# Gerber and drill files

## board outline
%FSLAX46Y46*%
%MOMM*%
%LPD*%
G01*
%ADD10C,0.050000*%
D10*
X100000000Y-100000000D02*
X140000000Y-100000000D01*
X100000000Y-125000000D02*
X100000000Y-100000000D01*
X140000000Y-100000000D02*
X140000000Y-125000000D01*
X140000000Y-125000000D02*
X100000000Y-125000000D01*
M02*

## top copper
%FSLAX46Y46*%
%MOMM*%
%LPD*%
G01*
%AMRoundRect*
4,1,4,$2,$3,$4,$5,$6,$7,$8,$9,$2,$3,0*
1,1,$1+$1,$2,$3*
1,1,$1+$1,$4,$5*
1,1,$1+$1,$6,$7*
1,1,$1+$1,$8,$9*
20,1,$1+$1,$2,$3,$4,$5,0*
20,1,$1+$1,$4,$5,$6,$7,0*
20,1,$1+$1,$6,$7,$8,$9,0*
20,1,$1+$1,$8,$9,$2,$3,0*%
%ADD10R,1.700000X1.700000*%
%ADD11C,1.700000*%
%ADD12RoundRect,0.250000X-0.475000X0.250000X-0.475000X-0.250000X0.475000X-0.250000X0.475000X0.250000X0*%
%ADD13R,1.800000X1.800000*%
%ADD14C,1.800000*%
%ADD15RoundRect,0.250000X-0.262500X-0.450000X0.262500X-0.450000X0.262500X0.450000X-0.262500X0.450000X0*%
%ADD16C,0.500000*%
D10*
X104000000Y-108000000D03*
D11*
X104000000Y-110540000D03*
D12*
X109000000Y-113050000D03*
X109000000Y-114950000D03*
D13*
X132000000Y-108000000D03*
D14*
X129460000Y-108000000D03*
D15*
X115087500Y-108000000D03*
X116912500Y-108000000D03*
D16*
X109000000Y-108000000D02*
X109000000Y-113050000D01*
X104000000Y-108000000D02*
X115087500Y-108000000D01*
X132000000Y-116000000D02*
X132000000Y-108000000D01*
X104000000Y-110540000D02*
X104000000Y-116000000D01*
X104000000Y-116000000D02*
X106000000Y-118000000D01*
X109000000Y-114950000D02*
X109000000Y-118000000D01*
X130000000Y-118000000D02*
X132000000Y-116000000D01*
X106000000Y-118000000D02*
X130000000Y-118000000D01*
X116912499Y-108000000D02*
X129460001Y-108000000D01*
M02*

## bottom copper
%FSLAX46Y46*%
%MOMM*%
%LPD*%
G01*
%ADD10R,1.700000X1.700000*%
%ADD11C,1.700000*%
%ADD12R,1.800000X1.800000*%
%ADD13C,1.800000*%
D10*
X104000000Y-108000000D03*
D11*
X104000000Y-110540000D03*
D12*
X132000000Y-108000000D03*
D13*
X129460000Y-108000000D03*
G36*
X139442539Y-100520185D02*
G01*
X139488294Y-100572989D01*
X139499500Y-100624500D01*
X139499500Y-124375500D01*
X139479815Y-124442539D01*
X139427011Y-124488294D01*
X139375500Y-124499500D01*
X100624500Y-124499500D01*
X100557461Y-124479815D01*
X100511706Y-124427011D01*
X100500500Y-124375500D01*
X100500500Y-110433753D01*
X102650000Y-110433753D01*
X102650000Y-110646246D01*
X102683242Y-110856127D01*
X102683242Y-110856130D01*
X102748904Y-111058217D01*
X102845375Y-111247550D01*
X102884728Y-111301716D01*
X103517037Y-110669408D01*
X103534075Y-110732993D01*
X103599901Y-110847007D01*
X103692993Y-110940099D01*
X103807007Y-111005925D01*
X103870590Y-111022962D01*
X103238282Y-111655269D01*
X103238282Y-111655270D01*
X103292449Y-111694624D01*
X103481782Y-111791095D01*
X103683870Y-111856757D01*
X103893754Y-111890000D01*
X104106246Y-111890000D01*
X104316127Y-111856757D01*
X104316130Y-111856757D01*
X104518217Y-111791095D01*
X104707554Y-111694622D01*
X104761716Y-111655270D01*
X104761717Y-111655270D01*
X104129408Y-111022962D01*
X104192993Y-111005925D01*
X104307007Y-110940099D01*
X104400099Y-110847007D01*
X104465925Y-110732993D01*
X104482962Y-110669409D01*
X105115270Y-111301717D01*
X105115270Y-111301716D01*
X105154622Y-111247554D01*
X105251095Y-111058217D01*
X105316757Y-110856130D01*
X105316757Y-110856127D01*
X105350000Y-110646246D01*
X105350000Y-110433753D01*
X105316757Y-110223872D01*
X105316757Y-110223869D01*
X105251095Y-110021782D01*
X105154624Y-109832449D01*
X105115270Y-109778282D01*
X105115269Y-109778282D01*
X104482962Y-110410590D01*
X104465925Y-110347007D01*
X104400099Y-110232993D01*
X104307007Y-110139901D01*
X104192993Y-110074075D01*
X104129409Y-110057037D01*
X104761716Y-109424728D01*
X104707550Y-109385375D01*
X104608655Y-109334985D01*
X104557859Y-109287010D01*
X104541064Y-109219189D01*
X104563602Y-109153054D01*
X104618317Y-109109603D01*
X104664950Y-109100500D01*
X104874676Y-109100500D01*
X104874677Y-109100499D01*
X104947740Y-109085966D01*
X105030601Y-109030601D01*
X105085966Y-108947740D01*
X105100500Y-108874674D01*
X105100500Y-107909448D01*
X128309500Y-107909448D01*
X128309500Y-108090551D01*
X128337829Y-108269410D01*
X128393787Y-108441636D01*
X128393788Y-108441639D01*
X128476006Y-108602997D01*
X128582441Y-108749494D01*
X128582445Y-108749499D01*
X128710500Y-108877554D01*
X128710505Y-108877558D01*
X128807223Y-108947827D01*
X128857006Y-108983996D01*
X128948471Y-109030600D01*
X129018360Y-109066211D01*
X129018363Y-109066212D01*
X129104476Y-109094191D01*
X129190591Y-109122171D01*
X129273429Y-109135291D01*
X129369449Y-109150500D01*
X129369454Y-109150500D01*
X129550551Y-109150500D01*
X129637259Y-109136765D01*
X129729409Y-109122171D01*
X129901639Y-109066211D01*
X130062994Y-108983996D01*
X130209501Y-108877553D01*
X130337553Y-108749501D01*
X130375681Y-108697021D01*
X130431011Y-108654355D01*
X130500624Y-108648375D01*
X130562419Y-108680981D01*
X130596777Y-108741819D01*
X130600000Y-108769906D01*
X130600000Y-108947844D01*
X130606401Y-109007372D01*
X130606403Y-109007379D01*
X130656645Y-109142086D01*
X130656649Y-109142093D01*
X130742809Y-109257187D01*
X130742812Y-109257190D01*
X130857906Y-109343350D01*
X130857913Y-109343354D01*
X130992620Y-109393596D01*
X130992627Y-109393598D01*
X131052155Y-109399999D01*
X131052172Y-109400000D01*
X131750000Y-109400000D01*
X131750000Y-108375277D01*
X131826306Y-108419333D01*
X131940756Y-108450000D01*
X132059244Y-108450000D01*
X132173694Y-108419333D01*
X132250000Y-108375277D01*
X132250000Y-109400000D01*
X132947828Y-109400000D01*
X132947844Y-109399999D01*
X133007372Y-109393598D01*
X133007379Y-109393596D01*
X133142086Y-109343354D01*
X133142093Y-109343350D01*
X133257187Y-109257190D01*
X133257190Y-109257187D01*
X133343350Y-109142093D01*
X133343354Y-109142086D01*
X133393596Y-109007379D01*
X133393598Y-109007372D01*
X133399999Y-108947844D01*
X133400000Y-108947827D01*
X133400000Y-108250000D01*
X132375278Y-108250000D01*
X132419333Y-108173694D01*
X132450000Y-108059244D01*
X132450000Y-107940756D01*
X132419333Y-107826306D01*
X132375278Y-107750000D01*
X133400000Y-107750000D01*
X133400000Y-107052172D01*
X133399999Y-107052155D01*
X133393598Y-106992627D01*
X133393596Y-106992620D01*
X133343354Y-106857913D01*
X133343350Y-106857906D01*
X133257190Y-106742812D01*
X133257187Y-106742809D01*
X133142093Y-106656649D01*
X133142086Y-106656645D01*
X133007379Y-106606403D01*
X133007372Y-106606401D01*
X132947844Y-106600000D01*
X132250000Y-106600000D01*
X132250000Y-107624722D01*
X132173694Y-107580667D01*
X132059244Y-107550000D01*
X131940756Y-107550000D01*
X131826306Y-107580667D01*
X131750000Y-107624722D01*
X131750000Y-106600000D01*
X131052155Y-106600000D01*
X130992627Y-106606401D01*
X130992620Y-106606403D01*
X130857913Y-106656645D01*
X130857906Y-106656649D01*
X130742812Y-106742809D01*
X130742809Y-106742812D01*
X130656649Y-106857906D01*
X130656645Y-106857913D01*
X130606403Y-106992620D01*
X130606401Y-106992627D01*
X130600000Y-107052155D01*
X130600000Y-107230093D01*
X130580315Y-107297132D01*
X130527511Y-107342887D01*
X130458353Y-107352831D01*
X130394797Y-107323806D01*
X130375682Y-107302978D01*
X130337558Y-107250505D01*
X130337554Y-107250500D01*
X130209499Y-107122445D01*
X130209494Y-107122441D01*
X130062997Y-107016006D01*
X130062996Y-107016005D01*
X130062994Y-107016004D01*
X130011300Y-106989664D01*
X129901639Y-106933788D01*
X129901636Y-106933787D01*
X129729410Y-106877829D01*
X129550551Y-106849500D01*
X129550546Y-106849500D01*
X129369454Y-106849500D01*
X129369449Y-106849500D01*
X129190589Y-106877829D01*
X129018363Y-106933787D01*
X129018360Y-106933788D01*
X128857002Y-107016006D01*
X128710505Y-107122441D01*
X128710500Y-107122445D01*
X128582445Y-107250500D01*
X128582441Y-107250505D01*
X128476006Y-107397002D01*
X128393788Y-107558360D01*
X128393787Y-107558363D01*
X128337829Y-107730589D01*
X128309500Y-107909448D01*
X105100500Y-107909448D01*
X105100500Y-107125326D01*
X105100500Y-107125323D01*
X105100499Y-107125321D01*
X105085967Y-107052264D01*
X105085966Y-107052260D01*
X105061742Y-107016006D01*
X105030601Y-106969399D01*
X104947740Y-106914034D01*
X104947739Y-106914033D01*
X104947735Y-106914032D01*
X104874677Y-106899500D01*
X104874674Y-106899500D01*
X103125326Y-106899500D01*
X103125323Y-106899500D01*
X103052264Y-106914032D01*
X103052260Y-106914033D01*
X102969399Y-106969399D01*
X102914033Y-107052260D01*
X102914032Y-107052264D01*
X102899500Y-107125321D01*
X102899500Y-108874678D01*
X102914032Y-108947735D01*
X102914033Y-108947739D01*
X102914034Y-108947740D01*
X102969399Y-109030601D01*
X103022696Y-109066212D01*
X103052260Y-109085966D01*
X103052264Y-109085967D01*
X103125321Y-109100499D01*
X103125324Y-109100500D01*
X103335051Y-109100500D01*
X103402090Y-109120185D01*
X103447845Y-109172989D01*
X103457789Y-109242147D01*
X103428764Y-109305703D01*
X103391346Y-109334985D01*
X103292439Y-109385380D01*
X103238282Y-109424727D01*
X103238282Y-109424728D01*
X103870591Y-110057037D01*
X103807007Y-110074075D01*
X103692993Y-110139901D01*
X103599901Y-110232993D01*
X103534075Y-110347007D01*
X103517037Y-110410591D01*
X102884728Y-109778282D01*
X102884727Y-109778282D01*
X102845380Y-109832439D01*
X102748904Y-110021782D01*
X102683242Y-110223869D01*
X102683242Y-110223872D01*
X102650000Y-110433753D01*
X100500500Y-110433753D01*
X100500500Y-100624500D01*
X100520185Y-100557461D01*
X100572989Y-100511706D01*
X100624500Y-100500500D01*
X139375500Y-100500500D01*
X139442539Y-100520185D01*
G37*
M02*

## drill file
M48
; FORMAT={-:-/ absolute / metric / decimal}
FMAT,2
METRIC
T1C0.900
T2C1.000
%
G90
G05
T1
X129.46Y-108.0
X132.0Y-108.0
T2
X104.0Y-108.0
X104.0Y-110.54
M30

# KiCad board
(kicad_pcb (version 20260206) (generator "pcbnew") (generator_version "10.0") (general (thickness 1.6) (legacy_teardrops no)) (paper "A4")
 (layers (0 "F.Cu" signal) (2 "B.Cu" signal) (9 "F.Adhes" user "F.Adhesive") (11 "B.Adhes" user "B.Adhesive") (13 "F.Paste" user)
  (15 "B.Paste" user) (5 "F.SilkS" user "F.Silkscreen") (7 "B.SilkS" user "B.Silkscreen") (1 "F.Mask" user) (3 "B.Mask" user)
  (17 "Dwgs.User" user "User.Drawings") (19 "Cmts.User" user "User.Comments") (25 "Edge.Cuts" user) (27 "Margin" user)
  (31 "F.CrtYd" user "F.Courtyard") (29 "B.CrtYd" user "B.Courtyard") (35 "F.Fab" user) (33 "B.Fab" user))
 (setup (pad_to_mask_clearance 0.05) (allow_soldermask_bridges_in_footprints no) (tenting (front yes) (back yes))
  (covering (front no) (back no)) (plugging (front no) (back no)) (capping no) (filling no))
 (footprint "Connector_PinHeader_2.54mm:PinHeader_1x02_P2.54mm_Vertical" (layer "F.Cu") (at 104 108)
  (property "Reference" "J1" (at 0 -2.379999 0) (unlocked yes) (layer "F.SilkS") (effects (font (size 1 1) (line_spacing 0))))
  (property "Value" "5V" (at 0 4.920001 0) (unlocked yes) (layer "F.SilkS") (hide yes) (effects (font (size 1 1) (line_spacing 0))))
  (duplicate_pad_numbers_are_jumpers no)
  (pad "1" thru_hole rect (at 0 0) (size 1.7 1.7) (drill 1) (layers "*.Cu" "*.Mask") (remove_unused_layers no) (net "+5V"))
  (pad "2" thru_hole circle (at 0 2.54) (size 1.7 1.7) (drill 1) (layers "*.Cu" "*.Mask") (remove_unused_layers no) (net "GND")))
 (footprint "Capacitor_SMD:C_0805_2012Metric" (layer "F.Cu") (at 109 114 -90)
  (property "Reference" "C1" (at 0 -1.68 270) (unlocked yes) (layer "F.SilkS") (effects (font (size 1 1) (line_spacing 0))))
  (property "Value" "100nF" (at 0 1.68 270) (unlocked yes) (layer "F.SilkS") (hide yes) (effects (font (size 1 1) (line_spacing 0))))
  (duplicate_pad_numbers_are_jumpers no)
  (pad "1" smd roundrect (at -0.95 0 270) (size 1 1.45) (layers "F.Cu" "F.Mask" "F.Paste") (roundrect_rratio 0.25) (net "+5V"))
  (pad "2" smd roundrect (at 0.95 0 270) (size 1 1.45) (layers "F.Cu" "F.Mask" "F.Paste") (roundrect_rratio 0.25) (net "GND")))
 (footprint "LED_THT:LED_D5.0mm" (layer "F.Cu") (at 132 108 180)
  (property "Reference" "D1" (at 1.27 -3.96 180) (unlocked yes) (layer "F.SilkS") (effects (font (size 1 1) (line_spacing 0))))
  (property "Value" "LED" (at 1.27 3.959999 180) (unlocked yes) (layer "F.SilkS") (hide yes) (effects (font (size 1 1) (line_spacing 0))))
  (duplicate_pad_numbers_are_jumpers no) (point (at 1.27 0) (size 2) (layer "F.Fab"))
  (pad "1" thru_hole rect (at 0 0 180) (size 1.8 1.8) (drill 0.9) (layers "*.Cu" "*.Mask") (remove_unused_layers no) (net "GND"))
  (pad "2" thru_hole circle (at 2.54 0 180) (size 1.8 1.8) (drill 0.9) (layers "*.Cu" "*.Mask") (remove_unused_layers no) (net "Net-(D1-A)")))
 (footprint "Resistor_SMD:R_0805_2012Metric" (layer "F.Cu") (at 116 108)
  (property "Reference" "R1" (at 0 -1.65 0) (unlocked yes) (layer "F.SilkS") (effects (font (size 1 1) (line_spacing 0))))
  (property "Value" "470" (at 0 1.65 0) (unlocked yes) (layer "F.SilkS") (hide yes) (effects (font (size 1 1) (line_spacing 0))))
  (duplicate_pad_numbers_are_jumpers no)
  (pad "1" smd roundrect (at -0.9125 0) (size 1.025 1.4) (layers "F.Cu" "F.Mask" "F.Paste") (roundrect_rratio 0.243902) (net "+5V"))
  (pad "2" smd roundrect (at 0.9125 0) (size 1.025 1.4) (layers "F.Cu" "F.Mask" "F.Paste") (roundrect_rratio 0.243902) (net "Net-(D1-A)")))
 (gr_line (start 100 100) (end 140 100) (stroke (width 0.05) (type default)) (layer "Edge.Cuts"))
 (gr_line (start 100 125) (end 100 100) (stroke (width 0.05) (type default)) (layer "Edge.Cuts"))
 (gr_line (start 140 100) (end 140 125) (stroke (width 0.05) (type default)) (layer "Edge.Cuts"))
 (gr_line (start 140 125) (end 100 125) (stroke (width 0.05) (type default)) (layer "Edge.Cuts"))
 (segment (start 109 108) (end 109 113.05) (width 0.5) (layer "F.Cu") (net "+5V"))
 (segment (start 104 108) (end 115.0875 108) (width 0.5) (layer "F.Cu") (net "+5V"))
 (segment (start 132 116) (end 132 108) (width 0.5) (layer "F.Cu") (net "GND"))
 (segment (start 104 110.54) (end 104 116) (width 0.5) (layer "F.Cu") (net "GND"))
 (segment (start 104 116) (end 106 118) (width 0.5) (layer "F.Cu") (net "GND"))
 (segment (start 109 114.95) (end 109 118) (width 0.5) (layer "F.Cu") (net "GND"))
 (segment (start 130 118) (end 132 116) (width 0.5) (layer "F.Cu") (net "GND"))
 (segment (start 106 118) (end 130 118) (width 0.5) (layer "F.Cu") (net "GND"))
 (segment (start 116.912499 108) (end 129.460001 108) (width 0.5) (layer "F.Cu") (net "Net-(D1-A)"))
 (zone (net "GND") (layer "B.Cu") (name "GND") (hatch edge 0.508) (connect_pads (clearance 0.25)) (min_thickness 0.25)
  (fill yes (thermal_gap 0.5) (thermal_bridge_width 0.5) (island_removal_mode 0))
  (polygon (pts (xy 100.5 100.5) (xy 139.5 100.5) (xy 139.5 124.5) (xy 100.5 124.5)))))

